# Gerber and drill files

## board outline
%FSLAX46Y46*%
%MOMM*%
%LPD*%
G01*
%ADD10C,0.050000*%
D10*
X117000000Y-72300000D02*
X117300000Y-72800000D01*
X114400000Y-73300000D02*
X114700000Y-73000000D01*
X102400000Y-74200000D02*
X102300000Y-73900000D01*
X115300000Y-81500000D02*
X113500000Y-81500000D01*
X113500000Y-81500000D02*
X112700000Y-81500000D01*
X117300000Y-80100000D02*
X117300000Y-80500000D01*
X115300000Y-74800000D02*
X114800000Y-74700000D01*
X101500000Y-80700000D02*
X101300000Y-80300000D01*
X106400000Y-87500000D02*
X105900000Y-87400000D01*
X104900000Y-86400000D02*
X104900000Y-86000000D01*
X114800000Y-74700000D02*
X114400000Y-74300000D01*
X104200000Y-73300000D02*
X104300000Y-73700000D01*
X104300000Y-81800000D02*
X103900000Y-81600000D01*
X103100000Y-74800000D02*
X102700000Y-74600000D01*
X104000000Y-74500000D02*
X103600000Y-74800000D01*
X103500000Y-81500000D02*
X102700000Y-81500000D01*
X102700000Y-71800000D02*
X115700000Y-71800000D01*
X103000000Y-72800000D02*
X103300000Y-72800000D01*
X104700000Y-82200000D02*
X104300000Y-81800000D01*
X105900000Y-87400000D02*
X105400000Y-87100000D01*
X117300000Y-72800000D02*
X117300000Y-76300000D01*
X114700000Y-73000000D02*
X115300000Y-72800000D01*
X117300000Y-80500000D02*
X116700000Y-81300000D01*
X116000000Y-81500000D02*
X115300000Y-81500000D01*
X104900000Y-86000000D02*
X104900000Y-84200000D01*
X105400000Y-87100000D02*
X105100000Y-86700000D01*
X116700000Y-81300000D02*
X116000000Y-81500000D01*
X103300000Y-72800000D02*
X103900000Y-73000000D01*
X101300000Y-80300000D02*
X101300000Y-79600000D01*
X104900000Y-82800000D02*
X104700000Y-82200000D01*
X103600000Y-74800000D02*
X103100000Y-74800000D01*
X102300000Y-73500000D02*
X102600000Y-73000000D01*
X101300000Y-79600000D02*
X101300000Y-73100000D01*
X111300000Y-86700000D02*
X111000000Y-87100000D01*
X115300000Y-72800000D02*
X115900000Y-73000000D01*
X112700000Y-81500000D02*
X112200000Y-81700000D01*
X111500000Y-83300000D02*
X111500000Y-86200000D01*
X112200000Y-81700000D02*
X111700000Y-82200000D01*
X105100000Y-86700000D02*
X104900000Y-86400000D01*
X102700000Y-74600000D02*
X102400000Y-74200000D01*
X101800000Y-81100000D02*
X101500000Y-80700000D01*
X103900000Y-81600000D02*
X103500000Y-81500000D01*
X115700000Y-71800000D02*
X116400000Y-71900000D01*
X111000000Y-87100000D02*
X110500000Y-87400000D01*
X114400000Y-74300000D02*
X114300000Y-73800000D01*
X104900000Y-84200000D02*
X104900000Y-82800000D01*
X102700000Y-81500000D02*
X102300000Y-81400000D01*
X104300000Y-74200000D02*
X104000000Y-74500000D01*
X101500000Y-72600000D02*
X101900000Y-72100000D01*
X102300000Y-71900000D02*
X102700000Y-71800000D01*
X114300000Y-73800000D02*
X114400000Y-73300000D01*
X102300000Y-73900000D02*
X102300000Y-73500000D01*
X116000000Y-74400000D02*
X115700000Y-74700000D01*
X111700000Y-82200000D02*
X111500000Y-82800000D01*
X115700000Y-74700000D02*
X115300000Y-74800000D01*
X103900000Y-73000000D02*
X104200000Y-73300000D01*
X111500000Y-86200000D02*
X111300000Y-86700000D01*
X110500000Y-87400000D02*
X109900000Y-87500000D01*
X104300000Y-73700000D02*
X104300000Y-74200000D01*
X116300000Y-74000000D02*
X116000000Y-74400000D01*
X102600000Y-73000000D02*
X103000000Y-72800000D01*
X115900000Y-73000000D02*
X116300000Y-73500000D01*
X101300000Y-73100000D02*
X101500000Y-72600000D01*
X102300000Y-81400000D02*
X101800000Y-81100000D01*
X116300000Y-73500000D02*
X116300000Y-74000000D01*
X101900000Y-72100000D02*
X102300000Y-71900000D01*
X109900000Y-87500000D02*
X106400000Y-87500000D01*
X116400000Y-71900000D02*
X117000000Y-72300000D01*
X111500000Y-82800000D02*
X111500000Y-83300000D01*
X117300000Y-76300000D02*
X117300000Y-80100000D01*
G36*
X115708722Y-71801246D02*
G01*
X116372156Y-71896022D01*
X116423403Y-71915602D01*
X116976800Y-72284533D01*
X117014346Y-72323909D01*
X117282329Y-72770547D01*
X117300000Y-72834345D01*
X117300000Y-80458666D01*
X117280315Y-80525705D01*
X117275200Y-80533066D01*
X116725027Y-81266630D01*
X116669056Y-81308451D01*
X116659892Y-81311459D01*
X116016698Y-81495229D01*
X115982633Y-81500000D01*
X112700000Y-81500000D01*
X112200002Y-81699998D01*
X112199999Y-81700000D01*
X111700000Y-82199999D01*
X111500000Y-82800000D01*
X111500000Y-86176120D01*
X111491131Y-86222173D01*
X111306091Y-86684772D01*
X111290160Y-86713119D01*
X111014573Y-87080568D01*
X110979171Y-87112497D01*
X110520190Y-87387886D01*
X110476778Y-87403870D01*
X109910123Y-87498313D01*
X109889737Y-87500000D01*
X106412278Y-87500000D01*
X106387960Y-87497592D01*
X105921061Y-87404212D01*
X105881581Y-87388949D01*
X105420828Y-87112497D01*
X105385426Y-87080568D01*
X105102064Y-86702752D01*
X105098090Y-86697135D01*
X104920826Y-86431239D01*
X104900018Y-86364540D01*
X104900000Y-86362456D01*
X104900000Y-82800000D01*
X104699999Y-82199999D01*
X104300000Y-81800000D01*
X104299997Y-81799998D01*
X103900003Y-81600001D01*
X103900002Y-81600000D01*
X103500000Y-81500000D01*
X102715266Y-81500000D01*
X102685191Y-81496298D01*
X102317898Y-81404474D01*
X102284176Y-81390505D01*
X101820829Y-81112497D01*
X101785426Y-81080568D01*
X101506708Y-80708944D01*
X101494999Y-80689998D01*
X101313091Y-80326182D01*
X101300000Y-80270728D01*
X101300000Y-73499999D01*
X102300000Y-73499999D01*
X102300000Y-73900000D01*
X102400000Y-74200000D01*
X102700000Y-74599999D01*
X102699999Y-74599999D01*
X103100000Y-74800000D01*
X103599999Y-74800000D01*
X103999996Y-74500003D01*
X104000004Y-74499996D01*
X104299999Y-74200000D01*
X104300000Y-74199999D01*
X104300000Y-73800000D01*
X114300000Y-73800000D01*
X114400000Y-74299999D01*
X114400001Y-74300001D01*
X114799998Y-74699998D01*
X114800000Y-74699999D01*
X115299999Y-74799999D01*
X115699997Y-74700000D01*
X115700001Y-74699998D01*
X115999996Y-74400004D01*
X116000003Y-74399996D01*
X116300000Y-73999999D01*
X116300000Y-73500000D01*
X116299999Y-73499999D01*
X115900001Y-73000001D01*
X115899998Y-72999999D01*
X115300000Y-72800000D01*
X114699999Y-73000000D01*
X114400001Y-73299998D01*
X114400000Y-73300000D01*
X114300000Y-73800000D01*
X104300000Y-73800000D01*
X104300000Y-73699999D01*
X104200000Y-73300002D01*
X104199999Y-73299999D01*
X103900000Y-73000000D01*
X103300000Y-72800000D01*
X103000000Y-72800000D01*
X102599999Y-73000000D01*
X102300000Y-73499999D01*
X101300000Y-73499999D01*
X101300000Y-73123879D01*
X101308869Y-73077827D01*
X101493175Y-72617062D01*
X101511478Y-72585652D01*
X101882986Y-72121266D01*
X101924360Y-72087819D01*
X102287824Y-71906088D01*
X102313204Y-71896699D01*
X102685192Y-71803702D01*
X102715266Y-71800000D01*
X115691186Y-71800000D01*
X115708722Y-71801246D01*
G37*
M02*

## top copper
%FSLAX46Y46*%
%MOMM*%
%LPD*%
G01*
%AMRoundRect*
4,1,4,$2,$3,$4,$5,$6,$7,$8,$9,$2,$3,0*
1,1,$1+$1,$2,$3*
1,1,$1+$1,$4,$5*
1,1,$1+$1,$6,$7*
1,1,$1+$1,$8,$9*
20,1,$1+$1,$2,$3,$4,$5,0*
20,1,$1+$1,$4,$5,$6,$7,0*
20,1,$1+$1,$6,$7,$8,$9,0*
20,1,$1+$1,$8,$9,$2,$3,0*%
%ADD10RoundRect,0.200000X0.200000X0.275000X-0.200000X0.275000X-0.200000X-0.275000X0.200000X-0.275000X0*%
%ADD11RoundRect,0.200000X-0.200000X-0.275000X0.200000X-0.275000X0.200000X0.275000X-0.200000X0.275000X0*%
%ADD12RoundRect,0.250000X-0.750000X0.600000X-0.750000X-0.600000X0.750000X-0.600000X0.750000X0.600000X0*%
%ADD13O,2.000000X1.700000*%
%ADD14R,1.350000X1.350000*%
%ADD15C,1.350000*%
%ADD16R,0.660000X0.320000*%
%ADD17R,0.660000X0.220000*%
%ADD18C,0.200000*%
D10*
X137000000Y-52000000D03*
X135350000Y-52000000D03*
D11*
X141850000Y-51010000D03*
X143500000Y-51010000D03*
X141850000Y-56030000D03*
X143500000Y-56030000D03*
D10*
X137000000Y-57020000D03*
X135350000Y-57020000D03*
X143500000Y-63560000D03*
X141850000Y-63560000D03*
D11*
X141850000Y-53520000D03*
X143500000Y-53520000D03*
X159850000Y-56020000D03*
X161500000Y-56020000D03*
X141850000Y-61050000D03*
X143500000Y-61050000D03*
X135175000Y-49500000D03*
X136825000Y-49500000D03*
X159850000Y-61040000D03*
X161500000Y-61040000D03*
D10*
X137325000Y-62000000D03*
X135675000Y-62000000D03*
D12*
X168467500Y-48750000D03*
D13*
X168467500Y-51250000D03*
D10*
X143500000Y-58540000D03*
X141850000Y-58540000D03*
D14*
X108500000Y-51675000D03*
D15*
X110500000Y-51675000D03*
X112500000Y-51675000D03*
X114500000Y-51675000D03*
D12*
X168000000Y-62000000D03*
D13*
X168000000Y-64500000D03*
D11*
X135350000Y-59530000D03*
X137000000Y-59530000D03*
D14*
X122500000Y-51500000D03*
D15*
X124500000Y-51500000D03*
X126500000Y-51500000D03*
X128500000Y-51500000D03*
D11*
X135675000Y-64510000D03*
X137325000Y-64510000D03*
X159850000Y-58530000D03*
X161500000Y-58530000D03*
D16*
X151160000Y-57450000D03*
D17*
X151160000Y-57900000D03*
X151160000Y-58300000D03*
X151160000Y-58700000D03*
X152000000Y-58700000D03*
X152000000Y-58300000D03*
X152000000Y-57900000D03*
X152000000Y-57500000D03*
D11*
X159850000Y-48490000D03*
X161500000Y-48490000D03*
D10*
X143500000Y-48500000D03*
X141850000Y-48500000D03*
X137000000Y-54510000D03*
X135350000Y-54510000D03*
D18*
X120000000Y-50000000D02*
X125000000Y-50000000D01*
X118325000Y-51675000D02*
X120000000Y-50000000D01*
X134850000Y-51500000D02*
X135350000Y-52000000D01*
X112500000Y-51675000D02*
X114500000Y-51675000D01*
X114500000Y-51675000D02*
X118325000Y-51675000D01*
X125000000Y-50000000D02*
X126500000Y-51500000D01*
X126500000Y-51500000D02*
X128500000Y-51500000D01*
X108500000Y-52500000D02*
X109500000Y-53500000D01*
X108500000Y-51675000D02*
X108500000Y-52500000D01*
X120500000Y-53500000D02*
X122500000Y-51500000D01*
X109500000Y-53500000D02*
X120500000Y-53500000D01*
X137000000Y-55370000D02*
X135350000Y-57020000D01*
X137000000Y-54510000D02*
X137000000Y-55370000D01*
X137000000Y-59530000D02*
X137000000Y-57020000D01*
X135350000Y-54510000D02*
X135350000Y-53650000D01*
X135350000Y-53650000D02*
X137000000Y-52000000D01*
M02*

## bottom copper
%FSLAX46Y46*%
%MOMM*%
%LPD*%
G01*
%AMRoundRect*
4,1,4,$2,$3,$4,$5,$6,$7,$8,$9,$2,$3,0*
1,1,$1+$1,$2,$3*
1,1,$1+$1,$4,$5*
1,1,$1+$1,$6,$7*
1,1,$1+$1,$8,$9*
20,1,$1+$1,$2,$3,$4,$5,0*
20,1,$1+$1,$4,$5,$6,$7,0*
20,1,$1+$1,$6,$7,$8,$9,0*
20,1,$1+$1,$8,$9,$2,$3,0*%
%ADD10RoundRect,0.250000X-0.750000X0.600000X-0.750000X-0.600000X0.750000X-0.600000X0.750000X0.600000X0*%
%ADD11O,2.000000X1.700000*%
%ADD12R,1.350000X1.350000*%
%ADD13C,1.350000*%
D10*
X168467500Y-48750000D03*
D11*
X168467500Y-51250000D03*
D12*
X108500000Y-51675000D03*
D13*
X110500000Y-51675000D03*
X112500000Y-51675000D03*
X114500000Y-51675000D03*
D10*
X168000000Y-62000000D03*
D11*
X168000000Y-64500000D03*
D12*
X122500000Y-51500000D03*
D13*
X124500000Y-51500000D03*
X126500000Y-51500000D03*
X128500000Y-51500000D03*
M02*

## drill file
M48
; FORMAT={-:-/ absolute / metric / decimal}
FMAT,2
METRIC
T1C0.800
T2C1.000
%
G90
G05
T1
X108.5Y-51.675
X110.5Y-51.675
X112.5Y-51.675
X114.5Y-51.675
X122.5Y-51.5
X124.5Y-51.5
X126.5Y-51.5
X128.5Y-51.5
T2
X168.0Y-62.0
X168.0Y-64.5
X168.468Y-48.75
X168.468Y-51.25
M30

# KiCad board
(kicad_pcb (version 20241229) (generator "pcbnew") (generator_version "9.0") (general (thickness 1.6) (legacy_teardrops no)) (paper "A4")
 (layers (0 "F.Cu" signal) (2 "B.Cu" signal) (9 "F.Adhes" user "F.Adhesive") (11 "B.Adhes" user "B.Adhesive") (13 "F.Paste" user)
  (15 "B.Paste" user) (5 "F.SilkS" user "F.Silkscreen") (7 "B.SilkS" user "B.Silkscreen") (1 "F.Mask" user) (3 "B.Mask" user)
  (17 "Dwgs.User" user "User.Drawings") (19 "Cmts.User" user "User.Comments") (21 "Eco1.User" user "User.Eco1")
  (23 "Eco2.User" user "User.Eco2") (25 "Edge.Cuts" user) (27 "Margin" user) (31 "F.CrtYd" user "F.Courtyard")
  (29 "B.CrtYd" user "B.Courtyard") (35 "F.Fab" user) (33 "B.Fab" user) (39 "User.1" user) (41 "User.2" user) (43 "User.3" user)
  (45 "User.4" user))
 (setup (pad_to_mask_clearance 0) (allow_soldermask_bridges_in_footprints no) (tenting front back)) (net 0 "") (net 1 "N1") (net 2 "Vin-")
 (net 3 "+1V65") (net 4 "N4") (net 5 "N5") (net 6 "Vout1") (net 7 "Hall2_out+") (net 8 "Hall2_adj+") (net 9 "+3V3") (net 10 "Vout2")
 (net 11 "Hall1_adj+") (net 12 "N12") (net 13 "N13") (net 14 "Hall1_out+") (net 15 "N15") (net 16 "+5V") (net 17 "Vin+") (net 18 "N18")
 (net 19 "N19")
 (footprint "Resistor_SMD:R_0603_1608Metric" (layer "F.Cu") (at 136.175 52 180)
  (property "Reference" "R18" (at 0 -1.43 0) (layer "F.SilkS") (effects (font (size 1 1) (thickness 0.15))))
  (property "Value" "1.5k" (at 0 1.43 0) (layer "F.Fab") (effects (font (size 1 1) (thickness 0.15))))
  (pad "1" smd roundrect (at -0.825 0 180) (size 0.8 0.95) (layers "F.Cu" "F.Mask" "F.Paste") (roundrect_rratio 0.25) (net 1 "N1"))
  (pad "2" smd roundrect (at 0.825 0 180) (size 0.8 0.95) (layers "F.Cu" "F.Mask" "F.Paste") (roundrect_rratio 0.25) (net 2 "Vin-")))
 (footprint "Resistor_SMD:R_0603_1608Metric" (layer "F.Cu") (at 142.675 51.01)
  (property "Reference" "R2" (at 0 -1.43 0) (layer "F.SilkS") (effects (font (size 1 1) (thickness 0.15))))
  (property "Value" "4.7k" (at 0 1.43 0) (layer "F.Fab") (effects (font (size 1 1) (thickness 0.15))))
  (pad "1" smd roundrect (at -0.825 0) (size 0.8 0.95) (layers "F.Cu" "F.Mask" "F.Paste") (roundrect_rratio 0.25) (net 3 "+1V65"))
  (pad "2" smd roundrect (at 0.825 0) (size 0.8 0.95) (layers "F.Cu" "F.Mask" "F.Paste") (roundrect_rratio 0.25) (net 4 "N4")))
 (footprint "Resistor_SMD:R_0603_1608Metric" (layer "F.Cu") (at 142.675 56.03)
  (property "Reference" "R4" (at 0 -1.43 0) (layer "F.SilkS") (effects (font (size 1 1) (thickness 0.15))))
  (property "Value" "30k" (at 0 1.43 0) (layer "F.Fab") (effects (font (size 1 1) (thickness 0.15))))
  (pad "1" smd roundrect (at -0.825 0) (size 0.8 0.95) (layers "F.Cu" "F.Mask" "F.Paste") (roundrect_rratio 0.25) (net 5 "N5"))
  (pad "2" smd roundrect (at 0.825 0) (size 0.8 0.95) (layers "F.Cu" "F.Mask" "F.Paste") (roundrect_rratio 0.25) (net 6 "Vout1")))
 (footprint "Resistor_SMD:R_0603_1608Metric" (layer "F.Cu") (at 136.175 57.02 180)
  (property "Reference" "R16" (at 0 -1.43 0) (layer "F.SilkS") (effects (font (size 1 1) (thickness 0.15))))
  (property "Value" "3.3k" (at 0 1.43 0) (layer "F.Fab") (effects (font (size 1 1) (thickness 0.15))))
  (pad "1" smd roundrect (at -0.825 0 180) (size 0.8 0.95) (layers "F.Cu" "F.Mask" "F.Paste") (roundrect_rratio 0.25) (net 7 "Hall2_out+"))
  (pad "2" smd roundrect (at 0.825 0 180) (size 0.8 0.95) (layers "F.Cu" "F.Mask" "F.Paste") (roundrect_rratio 0.25) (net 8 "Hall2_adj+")))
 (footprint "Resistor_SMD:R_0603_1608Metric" (layer "F.Cu") (at 142.675 63.56 180)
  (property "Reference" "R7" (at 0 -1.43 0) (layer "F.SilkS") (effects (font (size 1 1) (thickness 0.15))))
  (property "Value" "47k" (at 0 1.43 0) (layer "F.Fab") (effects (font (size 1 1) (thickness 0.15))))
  (pad "1" smd roundrect (at -0.825 0 180) (size 0.8 0.95) (layers "F.Cu" "F.Mask" "F.Paste") (roundrect_rratio 0.25) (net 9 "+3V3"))
  (pad "2" smd roundrect (at 0.825 0 180) (size 0.8 0.95) (layers "F.Cu" "F.Mask" "F.Paste") (roundrect_rratio 0.25) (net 3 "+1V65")))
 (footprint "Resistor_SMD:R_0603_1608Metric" (layer "F.Cu") (at 142.675 53.52)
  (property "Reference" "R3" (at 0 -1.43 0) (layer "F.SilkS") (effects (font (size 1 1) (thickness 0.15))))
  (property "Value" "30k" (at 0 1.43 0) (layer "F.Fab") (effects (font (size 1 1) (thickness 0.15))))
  (pad "1" smd roundrect (at -0.825 0) (size 0.8 0.95) (layers "F.Cu" "F.Mask" "F.Paste") (roundrect_rratio 0.25) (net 4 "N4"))
  (pad "2" smd roundrect (at 0.825 0) (size 0.8 0.95) (layers "F.Cu" "F.Mask" "F.Paste") (roundrect_rratio 0.25) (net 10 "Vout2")))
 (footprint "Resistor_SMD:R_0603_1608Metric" (layer "F.Cu") (at 160.675 56.02)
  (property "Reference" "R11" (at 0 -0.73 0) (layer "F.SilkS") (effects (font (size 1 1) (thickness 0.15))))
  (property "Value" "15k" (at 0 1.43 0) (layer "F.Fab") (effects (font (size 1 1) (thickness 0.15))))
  (pad "1" smd roundrect (at -0.825 0) (size 0.8 0.95) (layers "F.Cu" "F.Mask" "F.Paste") (roundrect_rratio 0.25) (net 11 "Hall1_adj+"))
  (pad "2" smd roundrect (at 0.825 0) (size 0.8 0.95) (layers "F.Cu" "F.Mask" "F.Paste") (roundrect_rratio 0.25) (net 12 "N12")))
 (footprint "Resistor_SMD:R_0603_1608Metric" (layer "F.Cu") (at 142.675 61.05)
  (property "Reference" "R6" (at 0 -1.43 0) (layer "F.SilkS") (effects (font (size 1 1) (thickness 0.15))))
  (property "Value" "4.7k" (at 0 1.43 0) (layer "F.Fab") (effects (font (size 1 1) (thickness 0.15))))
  (pad "1" smd roundrect (at -0.825 0) (size 0.8 0.95) (layers "F.Cu" "F.Mask" "F.Paste") (roundrect_rratio 0.25) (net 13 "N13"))
  (pad "2" smd roundrect (at 0.825 0) (size 0.8 0.95) (layers "F.Cu" "F.Mask" "F.Paste") (roundrect_rratio 0.25) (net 11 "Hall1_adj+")))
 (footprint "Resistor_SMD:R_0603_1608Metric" (layer "F.Cu") (at 136 49.5)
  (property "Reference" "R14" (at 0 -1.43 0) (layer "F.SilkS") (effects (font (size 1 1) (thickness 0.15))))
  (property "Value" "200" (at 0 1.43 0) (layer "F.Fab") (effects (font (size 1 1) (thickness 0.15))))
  (pad "1" smd roundrect (at -0.825 0) (size 0.8 0.95) (layers "F.Cu" "F.Mask" "F.Paste") (roundrect_rratio 0.25) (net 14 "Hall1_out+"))
  (pad "2" smd roundrect (at 0.825 0) (size 0.8 0.95) (layers "F.Cu" "F.Mask" "F.Paste") (roundrect_rratio 0.25) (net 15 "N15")))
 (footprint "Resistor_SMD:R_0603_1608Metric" (layer "F.Cu") (at 160.675 61.04)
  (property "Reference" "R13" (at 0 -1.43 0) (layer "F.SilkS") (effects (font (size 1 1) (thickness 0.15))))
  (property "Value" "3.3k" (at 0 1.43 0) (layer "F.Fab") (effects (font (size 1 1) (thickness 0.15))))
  (pad "1" smd roundrect (at -0.825 0) (size 0.8 0.95) (layers "F.Cu" "F.Mask" "F.Paste") (roundrect_rratio 0.25) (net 14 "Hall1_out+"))
  (pad "2" smd roundrect (at 0.825 0) (size 0.8 0.95) (layers "F.Cu" "F.Mask" "F.Paste") (roundrect_rratio 0.25) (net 11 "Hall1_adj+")))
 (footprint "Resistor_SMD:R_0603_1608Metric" (layer "F.Cu") (at 136.5 62 180)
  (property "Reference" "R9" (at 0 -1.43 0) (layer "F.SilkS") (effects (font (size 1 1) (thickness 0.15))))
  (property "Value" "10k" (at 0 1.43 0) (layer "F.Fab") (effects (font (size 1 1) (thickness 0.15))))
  (pad "1" smd roundrect (at -0.825 0 180) (size 0.8 0.95) (layers "F.Cu" "F.Mask" "F.Paste") (roundrect_rratio 0.25) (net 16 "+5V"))
  (pad "2" smd roundrect (at 0.825 0 180) (size 0.8 0.95) (layers "F.Cu" "F.Mask" "F.Paste") (roundrect_rratio 0.25) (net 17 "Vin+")))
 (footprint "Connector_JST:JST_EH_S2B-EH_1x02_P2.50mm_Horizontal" (layer "F.Cu") (at 168.4675 48.75 -90)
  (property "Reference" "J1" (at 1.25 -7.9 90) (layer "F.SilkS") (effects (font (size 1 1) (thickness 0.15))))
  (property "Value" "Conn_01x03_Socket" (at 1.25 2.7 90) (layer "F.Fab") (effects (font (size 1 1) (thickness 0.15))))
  (pad "1" thru_hole roundrect (at 0 0 270) (size 1.7 2) (drill 1) (layers "*.Cu" "*.Mask") (remove_unused_layers no)
   (roundrect_rratio 0.147059) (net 16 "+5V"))
  (pad "2" thru_hole oval (at 2.5 0 270) (size 1.7 2) (drill 1) (layers "*.Cu" "*.Mask") (remove_unused_layers no) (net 9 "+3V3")))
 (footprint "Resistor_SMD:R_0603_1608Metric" (layer "F.Cu") (at 142.675 58.54 180)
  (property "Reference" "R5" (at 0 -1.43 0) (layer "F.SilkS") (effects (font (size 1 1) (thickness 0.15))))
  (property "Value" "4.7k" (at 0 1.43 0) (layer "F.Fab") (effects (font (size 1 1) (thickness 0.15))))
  (pad "1" smd roundrect (at -0.825 0 180) (size 0.8 0.95) (layers "F.Cu" "F.Mask" "F.Paste") (roundrect_rratio 0.25) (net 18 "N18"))
  (pad "2" smd roundrect (at 0.825 0 180) (size 0.8 0.95) (layers "F.Cu" "F.Mask" "F.Paste") (roundrect_rratio 0.25) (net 8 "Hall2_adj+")))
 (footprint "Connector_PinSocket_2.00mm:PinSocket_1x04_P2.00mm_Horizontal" (layer "F.Cu") (at 108.5 51.675 90)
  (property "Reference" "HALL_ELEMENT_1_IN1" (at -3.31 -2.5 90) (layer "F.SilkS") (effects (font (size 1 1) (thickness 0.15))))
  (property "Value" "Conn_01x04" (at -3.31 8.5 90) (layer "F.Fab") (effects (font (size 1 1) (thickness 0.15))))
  (pad "1" thru_hole rect (at 0 0 90) (size 1.35 1.35) (drill 0.8) (layers "*.Cu" "*.Mask") (remove_unused_layers no) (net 17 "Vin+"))
  (pad "2" thru_hole circle (at 0 2 90) (size 1.35 1.35) (drill 0.8) (layers "*.Cu" "*.Mask") (remove_unused_layers no)
   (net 14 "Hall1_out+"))
  (pad "3" thru_hole circle (at 0 4 90) (size 1.35 1.35) (drill 0.8) (layers "*.Cu" "*.Mask") (remove_unused_layers no) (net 2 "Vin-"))
  (pad "4" thru_hole circle (at 0 6 90) (size 1.35 1.35) (drill 0.8) (layers "*.Cu" "*.Mask") (remove_unused_layers no) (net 2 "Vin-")))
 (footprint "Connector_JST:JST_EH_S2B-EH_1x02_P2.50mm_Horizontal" (layer "F.Cu") (at 168 62 -90)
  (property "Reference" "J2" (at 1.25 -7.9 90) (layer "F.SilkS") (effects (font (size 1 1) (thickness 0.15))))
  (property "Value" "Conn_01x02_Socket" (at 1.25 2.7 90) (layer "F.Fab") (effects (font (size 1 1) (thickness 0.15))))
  (pad "1" thru_hole roundrect (at 0 0 270) (size 1.7 2) (drill 1) (layers "*.Cu" "*.Mask") (remove_unused_layers no)
   (roundrect_rratio 0.147059) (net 6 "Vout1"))
  (pad "2" thru_hole oval (at 2.5 0 270) (size 1.7 2) (drill 1) (layers "*.Cu" "*.Mask") (remove_unused_layers no) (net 10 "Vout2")))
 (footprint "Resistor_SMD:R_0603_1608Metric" (layer "F.Cu") (at 136.175 59.53)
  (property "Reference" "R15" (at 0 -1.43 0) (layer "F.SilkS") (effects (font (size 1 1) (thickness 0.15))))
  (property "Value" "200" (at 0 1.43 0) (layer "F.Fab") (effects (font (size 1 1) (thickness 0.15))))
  (pad "1" smd roundrect (at -0.825 0) (size 0.8 0.95) (layers "F.Cu" "F.Mask" "F.Paste") (roundrect_rratio 0.25) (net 7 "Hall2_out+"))
  (pad "2" smd roundrect (at 0.825 0) (size 0.8 0.95) (layers "F.Cu" "F.Mask" "F.Paste") (roundrect_rratio 0.25) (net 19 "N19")))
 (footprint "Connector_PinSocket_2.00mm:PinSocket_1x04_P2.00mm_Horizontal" (layer "F.Cu") (at 122.5 51.5 90)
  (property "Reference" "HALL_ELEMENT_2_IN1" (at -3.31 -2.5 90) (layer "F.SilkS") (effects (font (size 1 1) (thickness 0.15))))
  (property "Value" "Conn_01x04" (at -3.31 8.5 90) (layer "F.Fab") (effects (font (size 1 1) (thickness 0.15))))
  (pad "1" thru_hole rect (at 0 0 90) (size 1.35 1.35) (drill 0.8) (layers "*.Cu" "*.Mask") (remove_unused_layers no) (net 17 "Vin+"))
  (pad "2" thru_hole circle (at 0 2 90) (size 1.35 1.35) (drill 0.8) (layers "*.Cu" "*.Mask") (remove_unused_layers no) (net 7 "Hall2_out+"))
  (pad "3" thru_hole circle (at 0 4 90) (size 1.35 1.35) (drill 0.8) (layers "*.Cu" "*.Mask") (remove_unused_layers no) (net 2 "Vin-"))
  (pad "4" thru_hole circle (at 0 6 90) (size 1.35 1.35) (drill 0.8) (layers "*.Cu" "*.Mask") (remove_unused_layers no) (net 2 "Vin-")))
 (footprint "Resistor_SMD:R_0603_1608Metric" (layer "F.Cu") (at 136.5 64.51)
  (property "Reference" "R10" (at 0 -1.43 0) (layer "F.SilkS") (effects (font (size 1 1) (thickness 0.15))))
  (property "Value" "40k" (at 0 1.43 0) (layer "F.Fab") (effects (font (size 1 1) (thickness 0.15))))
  (pad "1" smd roundrect (at -0.825 0) (size 0.8 0.95) (layers "F.Cu" "F.Mask" "F.Paste") (roundrect_rratio 0.25) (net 17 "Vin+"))
  (pad "2" smd roundrect (at 0.825 0) (size 0.8 0.95) (layers "F.Cu" "F.Mask" "F.Paste") (roundrect_rratio 0.25) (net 2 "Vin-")))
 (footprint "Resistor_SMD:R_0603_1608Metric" (layer "F.Cu") (at 160.675 58.53)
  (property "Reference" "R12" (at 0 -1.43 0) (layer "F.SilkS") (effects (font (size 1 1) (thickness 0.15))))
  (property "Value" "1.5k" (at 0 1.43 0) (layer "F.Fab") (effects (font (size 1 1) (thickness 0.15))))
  (pad "1" smd roundrect (at -0.825 0) (size 0.8 0.95) (layers "F.Cu" "F.Mask" "F.Paste") (roundrect_rratio 0.25) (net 12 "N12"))
  (pad "2" smd roundrect (at 0.825 0) (size 0.8 0.95) (layers "F.Cu" "F.Mask" "F.Paste") (roundrect_rratio 0.25) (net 2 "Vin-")))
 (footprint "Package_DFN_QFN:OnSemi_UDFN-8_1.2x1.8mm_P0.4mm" (layer "F.Cu") (at 151.58 58.1)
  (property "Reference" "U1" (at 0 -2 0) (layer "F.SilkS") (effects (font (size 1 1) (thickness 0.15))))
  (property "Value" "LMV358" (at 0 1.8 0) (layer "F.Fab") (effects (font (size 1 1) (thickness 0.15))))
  (pad "1" smd rect (at -0.42 -0.65) (size 0.66 0.32) (layers "F.Cu" "F.Mask" "F.Paste") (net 6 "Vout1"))
  (pad "2" smd rect (at -0.42 -0.2) (size 0.66 0.22) (layers "F.Cu" "F.Mask" "F.Paste") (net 13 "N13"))
  (pad "3" smd rect (at -0.42 0.2) (size 0.66 0.22) (layers "F.Cu" "F.Mask" "F.Paste") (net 5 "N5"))
  (pad "4" smd rect (at -0.42 0.6) (size 0.66 0.22) (layers "F.Cu" "F.Mask" "F.Paste") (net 2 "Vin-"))
  (pad "5" smd rect (at 0.42 0.6) (size 0.66 0.22) (layers "F.Cu" "F.Mask" "F.Paste") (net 4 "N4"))
  (pad "6" smd rect (at 0.42 0.2) (size 0.66 0.22) (layers "F.Cu" "F.Mask" "F.Paste") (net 18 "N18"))
  (pad "7" smd rect (at 0.42 -0.2) (size 0.66 0.22) (layers "F.Cu" "F.Mask" "F.Paste") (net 10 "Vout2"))
  (pad "8" smd rect (at 0.42 -0.6) (size 0.66 0.22) (layers "F.Cu" "F.Mask" "F.Paste") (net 9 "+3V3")))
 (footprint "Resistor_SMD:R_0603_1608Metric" (layer "F.Cu") (at 160.675 48.49)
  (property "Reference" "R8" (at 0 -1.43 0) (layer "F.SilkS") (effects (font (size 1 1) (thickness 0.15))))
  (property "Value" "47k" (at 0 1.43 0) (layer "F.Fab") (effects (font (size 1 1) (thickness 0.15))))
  (pad "1" smd roundrect (at -0.825 0) (size 0.8 0.95) (layers "F.Cu" "F.Mask" "F.Paste") (roundrect_rratio 0.25) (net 3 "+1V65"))
  (pad "2" smd roundrect (at 0.825 0) (size 0.8 0.95) (layers "F.Cu" "F.Mask" "F.Paste") (roundrect_rratio 0.25) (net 2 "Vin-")))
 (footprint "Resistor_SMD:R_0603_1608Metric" (layer "F.Cu") (at 142.675 48.5 180)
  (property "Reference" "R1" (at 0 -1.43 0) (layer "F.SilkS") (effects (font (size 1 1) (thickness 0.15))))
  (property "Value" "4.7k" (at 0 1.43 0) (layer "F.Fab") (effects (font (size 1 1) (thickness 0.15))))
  (pad "1" smd roundrect (at -0.825 0 180) (size 0.8 0.95) (layers "F.Cu" "F.Mask" "F.Paste") (roundrect_rratio 0.25) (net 3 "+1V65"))
  (pad "2" smd roundrect (at 0.825 0 180) (size 0.8 0.95) (layers "F.Cu" "F.Mask" "F.Paste") (roundrect_rratio 0.25) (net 5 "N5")))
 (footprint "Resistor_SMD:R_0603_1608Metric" (layer "F.Cu") (at 136.175 54.51 180)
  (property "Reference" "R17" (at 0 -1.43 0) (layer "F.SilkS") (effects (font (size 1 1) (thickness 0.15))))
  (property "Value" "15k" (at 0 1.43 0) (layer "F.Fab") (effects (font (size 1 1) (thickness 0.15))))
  (pad "1" smd roundrect (at -0.825 0 180) (size 0.8 0.95) (layers "F.Cu" "F.Mask" "F.Paste") (roundrect_rratio 0.25) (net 8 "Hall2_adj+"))
  (pad "2" smd roundrect (at 0.825 0 180) (size 0.8 0.95) (layers "F.Cu" "F.Mask" "F.Paste") (roundrect_rratio 0.25) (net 1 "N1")))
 (gr_line (start 117 72.3) (end 117.3 72.8) (stroke (width 0.05) (type default)) (layer "Edge.Cuts"))
 (gr_line (start 114.4 73.3) (end 114.7 73) (stroke (width 0.05) (type default)) (layer "Edge.Cuts"))
 (gr_line (start 102.4 74.2) (end 102.3 73.9) (stroke (width 0.05) (type default)) (layer "Edge.Cuts"))
 (gr_line (start 115.3 81.5) (end 113.5 81.5) (stroke (width 0.05) (type default)) (layer "Edge.Cuts"))
 (gr_line (start 113.5 81.5) (end 112.7 81.5) (stroke (width 0.05) (type default)) (layer "Edge.Cuts"))
 (gr_line (start 117.3 80.1) (end 117.3 80.5) (stroke (width 0.05) (type default)) (layer "Edge.Cuts"))
 (gr_line (start 115.3 74.8) (end 114.8 74.7) (stroke (width 0.05) (type default)) (layer "Edge.Cuts"))
 (gr_line (start 101.5 80.7) (end 101.3 80.3) (stroke (width 0.05) (type default)) (layer "Edge.Cuts"))
 (gr_line (start 106.4 87.5) (end 105.9 87.4) (stroke (width 0.05) (type default)) (layer "Edge.Cuts"))
 (gr_line (start 104.9 86.4) (end 104.9 86) (stroke (width 0.05) (type default)) (layer "Edge.Cuts"))
 (gr_line (start 114.8 74.7) (end 114.4 74.3) (stroke (width 0.05) (type default)) (layer "Edge.Cuts"))
 (gr_line (start 104.2 73.3) (end 104.3 73.7) (stroke (width 0.05) (type default)) (layer "Edge.Cuts"))
 (gr_line (start 104.3 81.8) (end 103.9 81.6) (stroke (width 0.05) (type default)) (layer "Edge.Cuts"))
 (gr_line (start 103.1 74.8) (end 102.7 74.6) (stroke (width 0.05) (type default)) (layer "Edge.Cuts"))
 (gr_line (start 104 74.5) (end 103.6 74.8) (stroke (width 0.05) (type default)) (layer "Edge.Cuts"))
 (gr_line (start 103.5 81.5) (end 102.7 81.5) (stroke (width 0.05) (type default)) (layer "Edge.Cuts"))
 (gr_line (start 102.7 71.8) (end 115.7 71.8) (stroke (width 0.05) (type default)) (layer "Edge.Cuts"))
 (gr_line (start 103 72.8) (end 103.3 72.8) (stroke (width 0.05) (type default)) (layer "Edge.Cuts"))
 (gr_line (start 104.7 82.2) (end 104.3 81.8) (stroke (width 0.05) (type default)) (layer "Edge.Cuts"))
 (gr_line (start 105.9 87.4) (end 105.4 87.1) (stroke (width 0.05) (type default)) (layer "Edge.Cuts"))
 (gr_line (start 117.3 72.8) (end 117.3 76.3) (stroke (width 0.05) (type default)) (layer "Edge.Cuts"))
 (gr_line (start 114.7 73) (end 115.3 72.8) (stroke (width 0.05) (type default)) (layer "Edge.Cuts"))
 (gr_line (start 117.3 80.5) (end 116.7 81.3) (stroke (width 0.05) (type default)) (layer "Edge.Cuts"))
 (gr_line (start 116 81.5) (end 115.3 81.5) (stroke (width 0.05) (type default)) (layer "Edge.Cuts"))
 (gr_line (start 104.9 86) (end 104.9 84.2) (stroke (width 0.05) (type default)) (layer "Edge.Cuts"))
 (gr_line (start 105.4 87.1) (end 105.1 86.7) (stroke (width 0.05) (type default)) (layer "Edge.Cuts"))
 (gr_line (start 116.7 81.3) (end 116 81.5) (stroke (width 0.05) (type default)) (layer "Edge.Cuts"))
 (gr_line (start 103.3 72.8) (end 103.9 73) (stroke (width 0.05) (type default)) (layer "Edge.Cuts"))
 (gr_line (start 101.3 80.3) (end 101.3 79.6) (stroke (width 0.05) (type default)) (layer "Edge.Cuts"))
 (gr_line (start 104.9 82.8) (end 104.7 82.2) (stroke (width 0.05) (type default)) (layer "Edge.Cuts"))
 (gr_line (start 103.6 74.8) (end 103.1 74.8) (stroke (width 0.05) (type default)) (layer "Edge.Cuts"))
 (gr_line (start 102.3 73.5) (end 102.6 73) (stroke (width 0.05) (type default)) (layer "Edge.Cuts"))
 (gr_line (start 101.3 79.6) (end 101.3 73.1) (stroke (width 0.05) (type default)) (layer "Edge.Cuts"))
 (gr_line (start 111.3 86.7) (end 111 87.1) (stroke (width 0.05) (type default)) (layer "Edge.Cuts"))
 (gr_line (start 115.3 72.8) (end 115.9 73) (stroke (width 0.05) (type default)) (layer "Edge.Cuts"))
 (gr_line (start 112.7 81.5) (end 112.2 81.7) (stroke (width 0.05) (type default)) (layer "Edge.Cuts"))
 (gr_line (start 111.5 83.3) (end 111.5 86.2) (stroke (width 0.05) (type default)) (layer "Edge.Cuts"))
 (gr_line (start 112.2 81.7) (end 111.7 82.2) (stroke (width 0.05) (type default)) (layer "Edge.Cuts"))
 (gr_line (start 105.1 86.7) (end 104.9 86.4) (stroke (width 0.05) (type default)) (layer "Edge.Cuts"))
 (gr_line (start 102.7 74.6) (end 102.4 74.2) (stroke (width 0.05) (type default)) (layer "Edge.Cuts"))
 (gr_line (start 101.8 81.1) (end 101.5 80.7) (stroke (width 0.05) (type default)) (layer "Edge.Cuts"))
 (gr_line (start 103.9 81.6) (end 103.5 81.5) (stroke (width 0.05) (type default)) (layer "Edge.Cuts"))
 (gr_line (start 115.7 71.8) (end 116.4 71.9) (stroke (width 0.05) (type default)) (layer "Edge.Cuts"))
 (gr_line (start 111 87.1) (end 110.5 87.4) (stroke (width 0.05) (type default)) (layer "Edge.Cuts"))
 (gr_line (start 114.4 74.3) (end 114.3 73.8) (stroke (width 0.05) (type default)) (layer "Edge.Cuts"))
 (gr_line (start 104.9 84.2) (end 104.9 82.8) (stroke (width 0.05) (type default)) (layer "Edge.Cuts"))
 (gr_line (start 102.7 81.5) (end 102.3 81.4) (stroke (width 0.05) (type default)) (layer "Edge.Cuts"))
 (gr_line (start 104.3 74.2) (end 104 74.5) (stroke (width 0.05) (type default)) (layer "Edge.Cuts"))
 (gr_line (start 101.5 72.6) (end 101.9 72.1) (stroke (width 0.05) (type default)) (layer "Edge.Cuts"))
 (gr_line (start 102.3 71.9) (end 102.7 71.8) (stroke (width 0.05) (type default)) (layer "Edge.Cuts"))
 (gr_line (start 114.3 73.8) (end 114.4 73.3) (stroke (width 0.05) (type default)) (layer "Edge.Cuts"))
 (gr_line (start 102.3 73.9) (end 102.3 73.5) (stroke (width 0.05) (type default)) (layer "Edge.Cuts"))
 (gr_line (start 116 74.4) (end 115.7 74.7) (stroke (width 0.05) (type default)) (layer "Edge.Cuts"))
 (gr_line (start 111.7 82.2) (end 111.5 82.8) (stroke (width 0.05) (type default)) (layer "Edge.Cuts"))
 (gr_line (start 115.7 74.7) (end 115.3 74.8) (stroke (width 0.05) (type default)) (layer "Edge.Cuts"))
 (gr_line (start 103.9 73) (end 104.2 73.3) (stroke (width 0.05) (type default)) (layer "Edge.Cuts"))
 (gr_line (start 111.5 86.2) (end 111.3 86.7) (stroke (width 0.05) (type default)) (layer "Edge.Cuts"))
 (gr_line (start 110.5 87.4) (end 109.9 87.5) (stroke (width 0.05) (type default)) (layer "Edge.Cuts"))
 (gr_line (start 104.3 73.7) (end 104.3 74.2) (stroke (width 0.05) (type default)) (layer "Edge.Cuts"))
 (gr_line (start 116.3 74) (end 116 74.4) (stroke (width 0.05) (type default)) (layer "Edge.Cuts"))
 (gr_line (start 102.6 73) (end 103 72.8) (stroke (width 0.05) (type default)) (layer "Edge.Cuts"))
 (gr_line (start 115.9 73) (end 116.3 73.5) (stroke (width 0.05) (type default)) (layer "Edge.Cuts"))
 (gr_line (start 101.3 73.1) (end 101.5 72.6) (stroke (width 0.05) (type default)) (layer "Edge.Cuts"))
 (gr_line (start 102.3 81.4) (end 101.8 81.1) (stroke (width 0.05) (type default)) (layer "Edge.Cuts"))
 (gr_line (start 116.3 73.5) (end 116.3 74) (stroke (width 0.05) (type default)) (layer "Edge.Cuts"))
 (gr_line (start 101.9 72.1) (end 102.3 71.9) (stroke (width 0.05) (type default)) (layer "Edge.Cuts"))
 (gr_line (start 109.9 87.5) (end 106.4 87.5) (stroke (width 0.05) (type default)) (layer "Edge.Cuts"))
 (gr_line (start 116.4 71.9) (end 117 72.3) (stroke (width 0.05) (type default)) (layer "Edge.Cuts"))
 (gr_line (start 111.5 82.8) (end 111.5 83.3) (stroke (width 0.05) (type default)) (layer "Edge.Cuts"))
 (gr_line (start 117.3 76.3) (end 117.3 80.1) (stroke (width 0.05) (type default)) (layer "Edge.Cuts"))
 (segment (start 120 50) (end 125 50) (width 0.2) (layer "F.Cu") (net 2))
 (segment (start 118.325 51.675) (end 120 50) (width 0.2) (layer "F.Cu") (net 2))
 (segment (start 134.85 51.5) (end 135.35 52) (width 0.2) (layer "F.Cu") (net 2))
 (segment (start 112.5 51.675) (end 114.5 51.675) (width 0.2) (layer "F.Cu") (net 2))
 (segment (start 114.5 51.675) (end 118.325 51.675) (width 0.2) (layer "F.Cu") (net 2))
 (segment (start 125 50) (end 126.5 51.5) (width 0.2) (layer "F.Cu") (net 2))
 (segment (start 126.5 51.5) (end 128.5 51.5) (width 0.2) (layer "F.Cu") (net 2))
 (segment (start 108.5 52.5) (end 109.5 53.5) (width 0.2) (layer "F.Cu") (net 17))
 (segment (start 108.5 51.675) (end 108.5 52.5) (width 0.2) (layer "F.Cu") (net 17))
 (segment (start 120.5 53.5) (end 122.5 51.5) (width 0.2) (layer "F.Cu") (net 17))
 (segment (start 109.5 53.5) (end 120.5 53.5) (width 0.2) (layer "F.Cu") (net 17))
 (segment (start 137 55.37) (end 135.35 57.02) (width 0.2) (layer "F.Cu") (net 8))
 (segment (start 137 54.51) (end 137 55.37) (width 0.2) (layer "F.Cu") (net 8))
 (segment (start 137 59.53) (end 137 57.02) (width 0.2) (layer "F.Cu") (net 19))
 (segment (start 135.35 54.51) (end 135.35 53.65) (width 0.2) (layer "F.Cu") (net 1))
 (segment (start 135.35 53.65) (end 137 52) (width 0.2) (layer "F.Cu") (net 1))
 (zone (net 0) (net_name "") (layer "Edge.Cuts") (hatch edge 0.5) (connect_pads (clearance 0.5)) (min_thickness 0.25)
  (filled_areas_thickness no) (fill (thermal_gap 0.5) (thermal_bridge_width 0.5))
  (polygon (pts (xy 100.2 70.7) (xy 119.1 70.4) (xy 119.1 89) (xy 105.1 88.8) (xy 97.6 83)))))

